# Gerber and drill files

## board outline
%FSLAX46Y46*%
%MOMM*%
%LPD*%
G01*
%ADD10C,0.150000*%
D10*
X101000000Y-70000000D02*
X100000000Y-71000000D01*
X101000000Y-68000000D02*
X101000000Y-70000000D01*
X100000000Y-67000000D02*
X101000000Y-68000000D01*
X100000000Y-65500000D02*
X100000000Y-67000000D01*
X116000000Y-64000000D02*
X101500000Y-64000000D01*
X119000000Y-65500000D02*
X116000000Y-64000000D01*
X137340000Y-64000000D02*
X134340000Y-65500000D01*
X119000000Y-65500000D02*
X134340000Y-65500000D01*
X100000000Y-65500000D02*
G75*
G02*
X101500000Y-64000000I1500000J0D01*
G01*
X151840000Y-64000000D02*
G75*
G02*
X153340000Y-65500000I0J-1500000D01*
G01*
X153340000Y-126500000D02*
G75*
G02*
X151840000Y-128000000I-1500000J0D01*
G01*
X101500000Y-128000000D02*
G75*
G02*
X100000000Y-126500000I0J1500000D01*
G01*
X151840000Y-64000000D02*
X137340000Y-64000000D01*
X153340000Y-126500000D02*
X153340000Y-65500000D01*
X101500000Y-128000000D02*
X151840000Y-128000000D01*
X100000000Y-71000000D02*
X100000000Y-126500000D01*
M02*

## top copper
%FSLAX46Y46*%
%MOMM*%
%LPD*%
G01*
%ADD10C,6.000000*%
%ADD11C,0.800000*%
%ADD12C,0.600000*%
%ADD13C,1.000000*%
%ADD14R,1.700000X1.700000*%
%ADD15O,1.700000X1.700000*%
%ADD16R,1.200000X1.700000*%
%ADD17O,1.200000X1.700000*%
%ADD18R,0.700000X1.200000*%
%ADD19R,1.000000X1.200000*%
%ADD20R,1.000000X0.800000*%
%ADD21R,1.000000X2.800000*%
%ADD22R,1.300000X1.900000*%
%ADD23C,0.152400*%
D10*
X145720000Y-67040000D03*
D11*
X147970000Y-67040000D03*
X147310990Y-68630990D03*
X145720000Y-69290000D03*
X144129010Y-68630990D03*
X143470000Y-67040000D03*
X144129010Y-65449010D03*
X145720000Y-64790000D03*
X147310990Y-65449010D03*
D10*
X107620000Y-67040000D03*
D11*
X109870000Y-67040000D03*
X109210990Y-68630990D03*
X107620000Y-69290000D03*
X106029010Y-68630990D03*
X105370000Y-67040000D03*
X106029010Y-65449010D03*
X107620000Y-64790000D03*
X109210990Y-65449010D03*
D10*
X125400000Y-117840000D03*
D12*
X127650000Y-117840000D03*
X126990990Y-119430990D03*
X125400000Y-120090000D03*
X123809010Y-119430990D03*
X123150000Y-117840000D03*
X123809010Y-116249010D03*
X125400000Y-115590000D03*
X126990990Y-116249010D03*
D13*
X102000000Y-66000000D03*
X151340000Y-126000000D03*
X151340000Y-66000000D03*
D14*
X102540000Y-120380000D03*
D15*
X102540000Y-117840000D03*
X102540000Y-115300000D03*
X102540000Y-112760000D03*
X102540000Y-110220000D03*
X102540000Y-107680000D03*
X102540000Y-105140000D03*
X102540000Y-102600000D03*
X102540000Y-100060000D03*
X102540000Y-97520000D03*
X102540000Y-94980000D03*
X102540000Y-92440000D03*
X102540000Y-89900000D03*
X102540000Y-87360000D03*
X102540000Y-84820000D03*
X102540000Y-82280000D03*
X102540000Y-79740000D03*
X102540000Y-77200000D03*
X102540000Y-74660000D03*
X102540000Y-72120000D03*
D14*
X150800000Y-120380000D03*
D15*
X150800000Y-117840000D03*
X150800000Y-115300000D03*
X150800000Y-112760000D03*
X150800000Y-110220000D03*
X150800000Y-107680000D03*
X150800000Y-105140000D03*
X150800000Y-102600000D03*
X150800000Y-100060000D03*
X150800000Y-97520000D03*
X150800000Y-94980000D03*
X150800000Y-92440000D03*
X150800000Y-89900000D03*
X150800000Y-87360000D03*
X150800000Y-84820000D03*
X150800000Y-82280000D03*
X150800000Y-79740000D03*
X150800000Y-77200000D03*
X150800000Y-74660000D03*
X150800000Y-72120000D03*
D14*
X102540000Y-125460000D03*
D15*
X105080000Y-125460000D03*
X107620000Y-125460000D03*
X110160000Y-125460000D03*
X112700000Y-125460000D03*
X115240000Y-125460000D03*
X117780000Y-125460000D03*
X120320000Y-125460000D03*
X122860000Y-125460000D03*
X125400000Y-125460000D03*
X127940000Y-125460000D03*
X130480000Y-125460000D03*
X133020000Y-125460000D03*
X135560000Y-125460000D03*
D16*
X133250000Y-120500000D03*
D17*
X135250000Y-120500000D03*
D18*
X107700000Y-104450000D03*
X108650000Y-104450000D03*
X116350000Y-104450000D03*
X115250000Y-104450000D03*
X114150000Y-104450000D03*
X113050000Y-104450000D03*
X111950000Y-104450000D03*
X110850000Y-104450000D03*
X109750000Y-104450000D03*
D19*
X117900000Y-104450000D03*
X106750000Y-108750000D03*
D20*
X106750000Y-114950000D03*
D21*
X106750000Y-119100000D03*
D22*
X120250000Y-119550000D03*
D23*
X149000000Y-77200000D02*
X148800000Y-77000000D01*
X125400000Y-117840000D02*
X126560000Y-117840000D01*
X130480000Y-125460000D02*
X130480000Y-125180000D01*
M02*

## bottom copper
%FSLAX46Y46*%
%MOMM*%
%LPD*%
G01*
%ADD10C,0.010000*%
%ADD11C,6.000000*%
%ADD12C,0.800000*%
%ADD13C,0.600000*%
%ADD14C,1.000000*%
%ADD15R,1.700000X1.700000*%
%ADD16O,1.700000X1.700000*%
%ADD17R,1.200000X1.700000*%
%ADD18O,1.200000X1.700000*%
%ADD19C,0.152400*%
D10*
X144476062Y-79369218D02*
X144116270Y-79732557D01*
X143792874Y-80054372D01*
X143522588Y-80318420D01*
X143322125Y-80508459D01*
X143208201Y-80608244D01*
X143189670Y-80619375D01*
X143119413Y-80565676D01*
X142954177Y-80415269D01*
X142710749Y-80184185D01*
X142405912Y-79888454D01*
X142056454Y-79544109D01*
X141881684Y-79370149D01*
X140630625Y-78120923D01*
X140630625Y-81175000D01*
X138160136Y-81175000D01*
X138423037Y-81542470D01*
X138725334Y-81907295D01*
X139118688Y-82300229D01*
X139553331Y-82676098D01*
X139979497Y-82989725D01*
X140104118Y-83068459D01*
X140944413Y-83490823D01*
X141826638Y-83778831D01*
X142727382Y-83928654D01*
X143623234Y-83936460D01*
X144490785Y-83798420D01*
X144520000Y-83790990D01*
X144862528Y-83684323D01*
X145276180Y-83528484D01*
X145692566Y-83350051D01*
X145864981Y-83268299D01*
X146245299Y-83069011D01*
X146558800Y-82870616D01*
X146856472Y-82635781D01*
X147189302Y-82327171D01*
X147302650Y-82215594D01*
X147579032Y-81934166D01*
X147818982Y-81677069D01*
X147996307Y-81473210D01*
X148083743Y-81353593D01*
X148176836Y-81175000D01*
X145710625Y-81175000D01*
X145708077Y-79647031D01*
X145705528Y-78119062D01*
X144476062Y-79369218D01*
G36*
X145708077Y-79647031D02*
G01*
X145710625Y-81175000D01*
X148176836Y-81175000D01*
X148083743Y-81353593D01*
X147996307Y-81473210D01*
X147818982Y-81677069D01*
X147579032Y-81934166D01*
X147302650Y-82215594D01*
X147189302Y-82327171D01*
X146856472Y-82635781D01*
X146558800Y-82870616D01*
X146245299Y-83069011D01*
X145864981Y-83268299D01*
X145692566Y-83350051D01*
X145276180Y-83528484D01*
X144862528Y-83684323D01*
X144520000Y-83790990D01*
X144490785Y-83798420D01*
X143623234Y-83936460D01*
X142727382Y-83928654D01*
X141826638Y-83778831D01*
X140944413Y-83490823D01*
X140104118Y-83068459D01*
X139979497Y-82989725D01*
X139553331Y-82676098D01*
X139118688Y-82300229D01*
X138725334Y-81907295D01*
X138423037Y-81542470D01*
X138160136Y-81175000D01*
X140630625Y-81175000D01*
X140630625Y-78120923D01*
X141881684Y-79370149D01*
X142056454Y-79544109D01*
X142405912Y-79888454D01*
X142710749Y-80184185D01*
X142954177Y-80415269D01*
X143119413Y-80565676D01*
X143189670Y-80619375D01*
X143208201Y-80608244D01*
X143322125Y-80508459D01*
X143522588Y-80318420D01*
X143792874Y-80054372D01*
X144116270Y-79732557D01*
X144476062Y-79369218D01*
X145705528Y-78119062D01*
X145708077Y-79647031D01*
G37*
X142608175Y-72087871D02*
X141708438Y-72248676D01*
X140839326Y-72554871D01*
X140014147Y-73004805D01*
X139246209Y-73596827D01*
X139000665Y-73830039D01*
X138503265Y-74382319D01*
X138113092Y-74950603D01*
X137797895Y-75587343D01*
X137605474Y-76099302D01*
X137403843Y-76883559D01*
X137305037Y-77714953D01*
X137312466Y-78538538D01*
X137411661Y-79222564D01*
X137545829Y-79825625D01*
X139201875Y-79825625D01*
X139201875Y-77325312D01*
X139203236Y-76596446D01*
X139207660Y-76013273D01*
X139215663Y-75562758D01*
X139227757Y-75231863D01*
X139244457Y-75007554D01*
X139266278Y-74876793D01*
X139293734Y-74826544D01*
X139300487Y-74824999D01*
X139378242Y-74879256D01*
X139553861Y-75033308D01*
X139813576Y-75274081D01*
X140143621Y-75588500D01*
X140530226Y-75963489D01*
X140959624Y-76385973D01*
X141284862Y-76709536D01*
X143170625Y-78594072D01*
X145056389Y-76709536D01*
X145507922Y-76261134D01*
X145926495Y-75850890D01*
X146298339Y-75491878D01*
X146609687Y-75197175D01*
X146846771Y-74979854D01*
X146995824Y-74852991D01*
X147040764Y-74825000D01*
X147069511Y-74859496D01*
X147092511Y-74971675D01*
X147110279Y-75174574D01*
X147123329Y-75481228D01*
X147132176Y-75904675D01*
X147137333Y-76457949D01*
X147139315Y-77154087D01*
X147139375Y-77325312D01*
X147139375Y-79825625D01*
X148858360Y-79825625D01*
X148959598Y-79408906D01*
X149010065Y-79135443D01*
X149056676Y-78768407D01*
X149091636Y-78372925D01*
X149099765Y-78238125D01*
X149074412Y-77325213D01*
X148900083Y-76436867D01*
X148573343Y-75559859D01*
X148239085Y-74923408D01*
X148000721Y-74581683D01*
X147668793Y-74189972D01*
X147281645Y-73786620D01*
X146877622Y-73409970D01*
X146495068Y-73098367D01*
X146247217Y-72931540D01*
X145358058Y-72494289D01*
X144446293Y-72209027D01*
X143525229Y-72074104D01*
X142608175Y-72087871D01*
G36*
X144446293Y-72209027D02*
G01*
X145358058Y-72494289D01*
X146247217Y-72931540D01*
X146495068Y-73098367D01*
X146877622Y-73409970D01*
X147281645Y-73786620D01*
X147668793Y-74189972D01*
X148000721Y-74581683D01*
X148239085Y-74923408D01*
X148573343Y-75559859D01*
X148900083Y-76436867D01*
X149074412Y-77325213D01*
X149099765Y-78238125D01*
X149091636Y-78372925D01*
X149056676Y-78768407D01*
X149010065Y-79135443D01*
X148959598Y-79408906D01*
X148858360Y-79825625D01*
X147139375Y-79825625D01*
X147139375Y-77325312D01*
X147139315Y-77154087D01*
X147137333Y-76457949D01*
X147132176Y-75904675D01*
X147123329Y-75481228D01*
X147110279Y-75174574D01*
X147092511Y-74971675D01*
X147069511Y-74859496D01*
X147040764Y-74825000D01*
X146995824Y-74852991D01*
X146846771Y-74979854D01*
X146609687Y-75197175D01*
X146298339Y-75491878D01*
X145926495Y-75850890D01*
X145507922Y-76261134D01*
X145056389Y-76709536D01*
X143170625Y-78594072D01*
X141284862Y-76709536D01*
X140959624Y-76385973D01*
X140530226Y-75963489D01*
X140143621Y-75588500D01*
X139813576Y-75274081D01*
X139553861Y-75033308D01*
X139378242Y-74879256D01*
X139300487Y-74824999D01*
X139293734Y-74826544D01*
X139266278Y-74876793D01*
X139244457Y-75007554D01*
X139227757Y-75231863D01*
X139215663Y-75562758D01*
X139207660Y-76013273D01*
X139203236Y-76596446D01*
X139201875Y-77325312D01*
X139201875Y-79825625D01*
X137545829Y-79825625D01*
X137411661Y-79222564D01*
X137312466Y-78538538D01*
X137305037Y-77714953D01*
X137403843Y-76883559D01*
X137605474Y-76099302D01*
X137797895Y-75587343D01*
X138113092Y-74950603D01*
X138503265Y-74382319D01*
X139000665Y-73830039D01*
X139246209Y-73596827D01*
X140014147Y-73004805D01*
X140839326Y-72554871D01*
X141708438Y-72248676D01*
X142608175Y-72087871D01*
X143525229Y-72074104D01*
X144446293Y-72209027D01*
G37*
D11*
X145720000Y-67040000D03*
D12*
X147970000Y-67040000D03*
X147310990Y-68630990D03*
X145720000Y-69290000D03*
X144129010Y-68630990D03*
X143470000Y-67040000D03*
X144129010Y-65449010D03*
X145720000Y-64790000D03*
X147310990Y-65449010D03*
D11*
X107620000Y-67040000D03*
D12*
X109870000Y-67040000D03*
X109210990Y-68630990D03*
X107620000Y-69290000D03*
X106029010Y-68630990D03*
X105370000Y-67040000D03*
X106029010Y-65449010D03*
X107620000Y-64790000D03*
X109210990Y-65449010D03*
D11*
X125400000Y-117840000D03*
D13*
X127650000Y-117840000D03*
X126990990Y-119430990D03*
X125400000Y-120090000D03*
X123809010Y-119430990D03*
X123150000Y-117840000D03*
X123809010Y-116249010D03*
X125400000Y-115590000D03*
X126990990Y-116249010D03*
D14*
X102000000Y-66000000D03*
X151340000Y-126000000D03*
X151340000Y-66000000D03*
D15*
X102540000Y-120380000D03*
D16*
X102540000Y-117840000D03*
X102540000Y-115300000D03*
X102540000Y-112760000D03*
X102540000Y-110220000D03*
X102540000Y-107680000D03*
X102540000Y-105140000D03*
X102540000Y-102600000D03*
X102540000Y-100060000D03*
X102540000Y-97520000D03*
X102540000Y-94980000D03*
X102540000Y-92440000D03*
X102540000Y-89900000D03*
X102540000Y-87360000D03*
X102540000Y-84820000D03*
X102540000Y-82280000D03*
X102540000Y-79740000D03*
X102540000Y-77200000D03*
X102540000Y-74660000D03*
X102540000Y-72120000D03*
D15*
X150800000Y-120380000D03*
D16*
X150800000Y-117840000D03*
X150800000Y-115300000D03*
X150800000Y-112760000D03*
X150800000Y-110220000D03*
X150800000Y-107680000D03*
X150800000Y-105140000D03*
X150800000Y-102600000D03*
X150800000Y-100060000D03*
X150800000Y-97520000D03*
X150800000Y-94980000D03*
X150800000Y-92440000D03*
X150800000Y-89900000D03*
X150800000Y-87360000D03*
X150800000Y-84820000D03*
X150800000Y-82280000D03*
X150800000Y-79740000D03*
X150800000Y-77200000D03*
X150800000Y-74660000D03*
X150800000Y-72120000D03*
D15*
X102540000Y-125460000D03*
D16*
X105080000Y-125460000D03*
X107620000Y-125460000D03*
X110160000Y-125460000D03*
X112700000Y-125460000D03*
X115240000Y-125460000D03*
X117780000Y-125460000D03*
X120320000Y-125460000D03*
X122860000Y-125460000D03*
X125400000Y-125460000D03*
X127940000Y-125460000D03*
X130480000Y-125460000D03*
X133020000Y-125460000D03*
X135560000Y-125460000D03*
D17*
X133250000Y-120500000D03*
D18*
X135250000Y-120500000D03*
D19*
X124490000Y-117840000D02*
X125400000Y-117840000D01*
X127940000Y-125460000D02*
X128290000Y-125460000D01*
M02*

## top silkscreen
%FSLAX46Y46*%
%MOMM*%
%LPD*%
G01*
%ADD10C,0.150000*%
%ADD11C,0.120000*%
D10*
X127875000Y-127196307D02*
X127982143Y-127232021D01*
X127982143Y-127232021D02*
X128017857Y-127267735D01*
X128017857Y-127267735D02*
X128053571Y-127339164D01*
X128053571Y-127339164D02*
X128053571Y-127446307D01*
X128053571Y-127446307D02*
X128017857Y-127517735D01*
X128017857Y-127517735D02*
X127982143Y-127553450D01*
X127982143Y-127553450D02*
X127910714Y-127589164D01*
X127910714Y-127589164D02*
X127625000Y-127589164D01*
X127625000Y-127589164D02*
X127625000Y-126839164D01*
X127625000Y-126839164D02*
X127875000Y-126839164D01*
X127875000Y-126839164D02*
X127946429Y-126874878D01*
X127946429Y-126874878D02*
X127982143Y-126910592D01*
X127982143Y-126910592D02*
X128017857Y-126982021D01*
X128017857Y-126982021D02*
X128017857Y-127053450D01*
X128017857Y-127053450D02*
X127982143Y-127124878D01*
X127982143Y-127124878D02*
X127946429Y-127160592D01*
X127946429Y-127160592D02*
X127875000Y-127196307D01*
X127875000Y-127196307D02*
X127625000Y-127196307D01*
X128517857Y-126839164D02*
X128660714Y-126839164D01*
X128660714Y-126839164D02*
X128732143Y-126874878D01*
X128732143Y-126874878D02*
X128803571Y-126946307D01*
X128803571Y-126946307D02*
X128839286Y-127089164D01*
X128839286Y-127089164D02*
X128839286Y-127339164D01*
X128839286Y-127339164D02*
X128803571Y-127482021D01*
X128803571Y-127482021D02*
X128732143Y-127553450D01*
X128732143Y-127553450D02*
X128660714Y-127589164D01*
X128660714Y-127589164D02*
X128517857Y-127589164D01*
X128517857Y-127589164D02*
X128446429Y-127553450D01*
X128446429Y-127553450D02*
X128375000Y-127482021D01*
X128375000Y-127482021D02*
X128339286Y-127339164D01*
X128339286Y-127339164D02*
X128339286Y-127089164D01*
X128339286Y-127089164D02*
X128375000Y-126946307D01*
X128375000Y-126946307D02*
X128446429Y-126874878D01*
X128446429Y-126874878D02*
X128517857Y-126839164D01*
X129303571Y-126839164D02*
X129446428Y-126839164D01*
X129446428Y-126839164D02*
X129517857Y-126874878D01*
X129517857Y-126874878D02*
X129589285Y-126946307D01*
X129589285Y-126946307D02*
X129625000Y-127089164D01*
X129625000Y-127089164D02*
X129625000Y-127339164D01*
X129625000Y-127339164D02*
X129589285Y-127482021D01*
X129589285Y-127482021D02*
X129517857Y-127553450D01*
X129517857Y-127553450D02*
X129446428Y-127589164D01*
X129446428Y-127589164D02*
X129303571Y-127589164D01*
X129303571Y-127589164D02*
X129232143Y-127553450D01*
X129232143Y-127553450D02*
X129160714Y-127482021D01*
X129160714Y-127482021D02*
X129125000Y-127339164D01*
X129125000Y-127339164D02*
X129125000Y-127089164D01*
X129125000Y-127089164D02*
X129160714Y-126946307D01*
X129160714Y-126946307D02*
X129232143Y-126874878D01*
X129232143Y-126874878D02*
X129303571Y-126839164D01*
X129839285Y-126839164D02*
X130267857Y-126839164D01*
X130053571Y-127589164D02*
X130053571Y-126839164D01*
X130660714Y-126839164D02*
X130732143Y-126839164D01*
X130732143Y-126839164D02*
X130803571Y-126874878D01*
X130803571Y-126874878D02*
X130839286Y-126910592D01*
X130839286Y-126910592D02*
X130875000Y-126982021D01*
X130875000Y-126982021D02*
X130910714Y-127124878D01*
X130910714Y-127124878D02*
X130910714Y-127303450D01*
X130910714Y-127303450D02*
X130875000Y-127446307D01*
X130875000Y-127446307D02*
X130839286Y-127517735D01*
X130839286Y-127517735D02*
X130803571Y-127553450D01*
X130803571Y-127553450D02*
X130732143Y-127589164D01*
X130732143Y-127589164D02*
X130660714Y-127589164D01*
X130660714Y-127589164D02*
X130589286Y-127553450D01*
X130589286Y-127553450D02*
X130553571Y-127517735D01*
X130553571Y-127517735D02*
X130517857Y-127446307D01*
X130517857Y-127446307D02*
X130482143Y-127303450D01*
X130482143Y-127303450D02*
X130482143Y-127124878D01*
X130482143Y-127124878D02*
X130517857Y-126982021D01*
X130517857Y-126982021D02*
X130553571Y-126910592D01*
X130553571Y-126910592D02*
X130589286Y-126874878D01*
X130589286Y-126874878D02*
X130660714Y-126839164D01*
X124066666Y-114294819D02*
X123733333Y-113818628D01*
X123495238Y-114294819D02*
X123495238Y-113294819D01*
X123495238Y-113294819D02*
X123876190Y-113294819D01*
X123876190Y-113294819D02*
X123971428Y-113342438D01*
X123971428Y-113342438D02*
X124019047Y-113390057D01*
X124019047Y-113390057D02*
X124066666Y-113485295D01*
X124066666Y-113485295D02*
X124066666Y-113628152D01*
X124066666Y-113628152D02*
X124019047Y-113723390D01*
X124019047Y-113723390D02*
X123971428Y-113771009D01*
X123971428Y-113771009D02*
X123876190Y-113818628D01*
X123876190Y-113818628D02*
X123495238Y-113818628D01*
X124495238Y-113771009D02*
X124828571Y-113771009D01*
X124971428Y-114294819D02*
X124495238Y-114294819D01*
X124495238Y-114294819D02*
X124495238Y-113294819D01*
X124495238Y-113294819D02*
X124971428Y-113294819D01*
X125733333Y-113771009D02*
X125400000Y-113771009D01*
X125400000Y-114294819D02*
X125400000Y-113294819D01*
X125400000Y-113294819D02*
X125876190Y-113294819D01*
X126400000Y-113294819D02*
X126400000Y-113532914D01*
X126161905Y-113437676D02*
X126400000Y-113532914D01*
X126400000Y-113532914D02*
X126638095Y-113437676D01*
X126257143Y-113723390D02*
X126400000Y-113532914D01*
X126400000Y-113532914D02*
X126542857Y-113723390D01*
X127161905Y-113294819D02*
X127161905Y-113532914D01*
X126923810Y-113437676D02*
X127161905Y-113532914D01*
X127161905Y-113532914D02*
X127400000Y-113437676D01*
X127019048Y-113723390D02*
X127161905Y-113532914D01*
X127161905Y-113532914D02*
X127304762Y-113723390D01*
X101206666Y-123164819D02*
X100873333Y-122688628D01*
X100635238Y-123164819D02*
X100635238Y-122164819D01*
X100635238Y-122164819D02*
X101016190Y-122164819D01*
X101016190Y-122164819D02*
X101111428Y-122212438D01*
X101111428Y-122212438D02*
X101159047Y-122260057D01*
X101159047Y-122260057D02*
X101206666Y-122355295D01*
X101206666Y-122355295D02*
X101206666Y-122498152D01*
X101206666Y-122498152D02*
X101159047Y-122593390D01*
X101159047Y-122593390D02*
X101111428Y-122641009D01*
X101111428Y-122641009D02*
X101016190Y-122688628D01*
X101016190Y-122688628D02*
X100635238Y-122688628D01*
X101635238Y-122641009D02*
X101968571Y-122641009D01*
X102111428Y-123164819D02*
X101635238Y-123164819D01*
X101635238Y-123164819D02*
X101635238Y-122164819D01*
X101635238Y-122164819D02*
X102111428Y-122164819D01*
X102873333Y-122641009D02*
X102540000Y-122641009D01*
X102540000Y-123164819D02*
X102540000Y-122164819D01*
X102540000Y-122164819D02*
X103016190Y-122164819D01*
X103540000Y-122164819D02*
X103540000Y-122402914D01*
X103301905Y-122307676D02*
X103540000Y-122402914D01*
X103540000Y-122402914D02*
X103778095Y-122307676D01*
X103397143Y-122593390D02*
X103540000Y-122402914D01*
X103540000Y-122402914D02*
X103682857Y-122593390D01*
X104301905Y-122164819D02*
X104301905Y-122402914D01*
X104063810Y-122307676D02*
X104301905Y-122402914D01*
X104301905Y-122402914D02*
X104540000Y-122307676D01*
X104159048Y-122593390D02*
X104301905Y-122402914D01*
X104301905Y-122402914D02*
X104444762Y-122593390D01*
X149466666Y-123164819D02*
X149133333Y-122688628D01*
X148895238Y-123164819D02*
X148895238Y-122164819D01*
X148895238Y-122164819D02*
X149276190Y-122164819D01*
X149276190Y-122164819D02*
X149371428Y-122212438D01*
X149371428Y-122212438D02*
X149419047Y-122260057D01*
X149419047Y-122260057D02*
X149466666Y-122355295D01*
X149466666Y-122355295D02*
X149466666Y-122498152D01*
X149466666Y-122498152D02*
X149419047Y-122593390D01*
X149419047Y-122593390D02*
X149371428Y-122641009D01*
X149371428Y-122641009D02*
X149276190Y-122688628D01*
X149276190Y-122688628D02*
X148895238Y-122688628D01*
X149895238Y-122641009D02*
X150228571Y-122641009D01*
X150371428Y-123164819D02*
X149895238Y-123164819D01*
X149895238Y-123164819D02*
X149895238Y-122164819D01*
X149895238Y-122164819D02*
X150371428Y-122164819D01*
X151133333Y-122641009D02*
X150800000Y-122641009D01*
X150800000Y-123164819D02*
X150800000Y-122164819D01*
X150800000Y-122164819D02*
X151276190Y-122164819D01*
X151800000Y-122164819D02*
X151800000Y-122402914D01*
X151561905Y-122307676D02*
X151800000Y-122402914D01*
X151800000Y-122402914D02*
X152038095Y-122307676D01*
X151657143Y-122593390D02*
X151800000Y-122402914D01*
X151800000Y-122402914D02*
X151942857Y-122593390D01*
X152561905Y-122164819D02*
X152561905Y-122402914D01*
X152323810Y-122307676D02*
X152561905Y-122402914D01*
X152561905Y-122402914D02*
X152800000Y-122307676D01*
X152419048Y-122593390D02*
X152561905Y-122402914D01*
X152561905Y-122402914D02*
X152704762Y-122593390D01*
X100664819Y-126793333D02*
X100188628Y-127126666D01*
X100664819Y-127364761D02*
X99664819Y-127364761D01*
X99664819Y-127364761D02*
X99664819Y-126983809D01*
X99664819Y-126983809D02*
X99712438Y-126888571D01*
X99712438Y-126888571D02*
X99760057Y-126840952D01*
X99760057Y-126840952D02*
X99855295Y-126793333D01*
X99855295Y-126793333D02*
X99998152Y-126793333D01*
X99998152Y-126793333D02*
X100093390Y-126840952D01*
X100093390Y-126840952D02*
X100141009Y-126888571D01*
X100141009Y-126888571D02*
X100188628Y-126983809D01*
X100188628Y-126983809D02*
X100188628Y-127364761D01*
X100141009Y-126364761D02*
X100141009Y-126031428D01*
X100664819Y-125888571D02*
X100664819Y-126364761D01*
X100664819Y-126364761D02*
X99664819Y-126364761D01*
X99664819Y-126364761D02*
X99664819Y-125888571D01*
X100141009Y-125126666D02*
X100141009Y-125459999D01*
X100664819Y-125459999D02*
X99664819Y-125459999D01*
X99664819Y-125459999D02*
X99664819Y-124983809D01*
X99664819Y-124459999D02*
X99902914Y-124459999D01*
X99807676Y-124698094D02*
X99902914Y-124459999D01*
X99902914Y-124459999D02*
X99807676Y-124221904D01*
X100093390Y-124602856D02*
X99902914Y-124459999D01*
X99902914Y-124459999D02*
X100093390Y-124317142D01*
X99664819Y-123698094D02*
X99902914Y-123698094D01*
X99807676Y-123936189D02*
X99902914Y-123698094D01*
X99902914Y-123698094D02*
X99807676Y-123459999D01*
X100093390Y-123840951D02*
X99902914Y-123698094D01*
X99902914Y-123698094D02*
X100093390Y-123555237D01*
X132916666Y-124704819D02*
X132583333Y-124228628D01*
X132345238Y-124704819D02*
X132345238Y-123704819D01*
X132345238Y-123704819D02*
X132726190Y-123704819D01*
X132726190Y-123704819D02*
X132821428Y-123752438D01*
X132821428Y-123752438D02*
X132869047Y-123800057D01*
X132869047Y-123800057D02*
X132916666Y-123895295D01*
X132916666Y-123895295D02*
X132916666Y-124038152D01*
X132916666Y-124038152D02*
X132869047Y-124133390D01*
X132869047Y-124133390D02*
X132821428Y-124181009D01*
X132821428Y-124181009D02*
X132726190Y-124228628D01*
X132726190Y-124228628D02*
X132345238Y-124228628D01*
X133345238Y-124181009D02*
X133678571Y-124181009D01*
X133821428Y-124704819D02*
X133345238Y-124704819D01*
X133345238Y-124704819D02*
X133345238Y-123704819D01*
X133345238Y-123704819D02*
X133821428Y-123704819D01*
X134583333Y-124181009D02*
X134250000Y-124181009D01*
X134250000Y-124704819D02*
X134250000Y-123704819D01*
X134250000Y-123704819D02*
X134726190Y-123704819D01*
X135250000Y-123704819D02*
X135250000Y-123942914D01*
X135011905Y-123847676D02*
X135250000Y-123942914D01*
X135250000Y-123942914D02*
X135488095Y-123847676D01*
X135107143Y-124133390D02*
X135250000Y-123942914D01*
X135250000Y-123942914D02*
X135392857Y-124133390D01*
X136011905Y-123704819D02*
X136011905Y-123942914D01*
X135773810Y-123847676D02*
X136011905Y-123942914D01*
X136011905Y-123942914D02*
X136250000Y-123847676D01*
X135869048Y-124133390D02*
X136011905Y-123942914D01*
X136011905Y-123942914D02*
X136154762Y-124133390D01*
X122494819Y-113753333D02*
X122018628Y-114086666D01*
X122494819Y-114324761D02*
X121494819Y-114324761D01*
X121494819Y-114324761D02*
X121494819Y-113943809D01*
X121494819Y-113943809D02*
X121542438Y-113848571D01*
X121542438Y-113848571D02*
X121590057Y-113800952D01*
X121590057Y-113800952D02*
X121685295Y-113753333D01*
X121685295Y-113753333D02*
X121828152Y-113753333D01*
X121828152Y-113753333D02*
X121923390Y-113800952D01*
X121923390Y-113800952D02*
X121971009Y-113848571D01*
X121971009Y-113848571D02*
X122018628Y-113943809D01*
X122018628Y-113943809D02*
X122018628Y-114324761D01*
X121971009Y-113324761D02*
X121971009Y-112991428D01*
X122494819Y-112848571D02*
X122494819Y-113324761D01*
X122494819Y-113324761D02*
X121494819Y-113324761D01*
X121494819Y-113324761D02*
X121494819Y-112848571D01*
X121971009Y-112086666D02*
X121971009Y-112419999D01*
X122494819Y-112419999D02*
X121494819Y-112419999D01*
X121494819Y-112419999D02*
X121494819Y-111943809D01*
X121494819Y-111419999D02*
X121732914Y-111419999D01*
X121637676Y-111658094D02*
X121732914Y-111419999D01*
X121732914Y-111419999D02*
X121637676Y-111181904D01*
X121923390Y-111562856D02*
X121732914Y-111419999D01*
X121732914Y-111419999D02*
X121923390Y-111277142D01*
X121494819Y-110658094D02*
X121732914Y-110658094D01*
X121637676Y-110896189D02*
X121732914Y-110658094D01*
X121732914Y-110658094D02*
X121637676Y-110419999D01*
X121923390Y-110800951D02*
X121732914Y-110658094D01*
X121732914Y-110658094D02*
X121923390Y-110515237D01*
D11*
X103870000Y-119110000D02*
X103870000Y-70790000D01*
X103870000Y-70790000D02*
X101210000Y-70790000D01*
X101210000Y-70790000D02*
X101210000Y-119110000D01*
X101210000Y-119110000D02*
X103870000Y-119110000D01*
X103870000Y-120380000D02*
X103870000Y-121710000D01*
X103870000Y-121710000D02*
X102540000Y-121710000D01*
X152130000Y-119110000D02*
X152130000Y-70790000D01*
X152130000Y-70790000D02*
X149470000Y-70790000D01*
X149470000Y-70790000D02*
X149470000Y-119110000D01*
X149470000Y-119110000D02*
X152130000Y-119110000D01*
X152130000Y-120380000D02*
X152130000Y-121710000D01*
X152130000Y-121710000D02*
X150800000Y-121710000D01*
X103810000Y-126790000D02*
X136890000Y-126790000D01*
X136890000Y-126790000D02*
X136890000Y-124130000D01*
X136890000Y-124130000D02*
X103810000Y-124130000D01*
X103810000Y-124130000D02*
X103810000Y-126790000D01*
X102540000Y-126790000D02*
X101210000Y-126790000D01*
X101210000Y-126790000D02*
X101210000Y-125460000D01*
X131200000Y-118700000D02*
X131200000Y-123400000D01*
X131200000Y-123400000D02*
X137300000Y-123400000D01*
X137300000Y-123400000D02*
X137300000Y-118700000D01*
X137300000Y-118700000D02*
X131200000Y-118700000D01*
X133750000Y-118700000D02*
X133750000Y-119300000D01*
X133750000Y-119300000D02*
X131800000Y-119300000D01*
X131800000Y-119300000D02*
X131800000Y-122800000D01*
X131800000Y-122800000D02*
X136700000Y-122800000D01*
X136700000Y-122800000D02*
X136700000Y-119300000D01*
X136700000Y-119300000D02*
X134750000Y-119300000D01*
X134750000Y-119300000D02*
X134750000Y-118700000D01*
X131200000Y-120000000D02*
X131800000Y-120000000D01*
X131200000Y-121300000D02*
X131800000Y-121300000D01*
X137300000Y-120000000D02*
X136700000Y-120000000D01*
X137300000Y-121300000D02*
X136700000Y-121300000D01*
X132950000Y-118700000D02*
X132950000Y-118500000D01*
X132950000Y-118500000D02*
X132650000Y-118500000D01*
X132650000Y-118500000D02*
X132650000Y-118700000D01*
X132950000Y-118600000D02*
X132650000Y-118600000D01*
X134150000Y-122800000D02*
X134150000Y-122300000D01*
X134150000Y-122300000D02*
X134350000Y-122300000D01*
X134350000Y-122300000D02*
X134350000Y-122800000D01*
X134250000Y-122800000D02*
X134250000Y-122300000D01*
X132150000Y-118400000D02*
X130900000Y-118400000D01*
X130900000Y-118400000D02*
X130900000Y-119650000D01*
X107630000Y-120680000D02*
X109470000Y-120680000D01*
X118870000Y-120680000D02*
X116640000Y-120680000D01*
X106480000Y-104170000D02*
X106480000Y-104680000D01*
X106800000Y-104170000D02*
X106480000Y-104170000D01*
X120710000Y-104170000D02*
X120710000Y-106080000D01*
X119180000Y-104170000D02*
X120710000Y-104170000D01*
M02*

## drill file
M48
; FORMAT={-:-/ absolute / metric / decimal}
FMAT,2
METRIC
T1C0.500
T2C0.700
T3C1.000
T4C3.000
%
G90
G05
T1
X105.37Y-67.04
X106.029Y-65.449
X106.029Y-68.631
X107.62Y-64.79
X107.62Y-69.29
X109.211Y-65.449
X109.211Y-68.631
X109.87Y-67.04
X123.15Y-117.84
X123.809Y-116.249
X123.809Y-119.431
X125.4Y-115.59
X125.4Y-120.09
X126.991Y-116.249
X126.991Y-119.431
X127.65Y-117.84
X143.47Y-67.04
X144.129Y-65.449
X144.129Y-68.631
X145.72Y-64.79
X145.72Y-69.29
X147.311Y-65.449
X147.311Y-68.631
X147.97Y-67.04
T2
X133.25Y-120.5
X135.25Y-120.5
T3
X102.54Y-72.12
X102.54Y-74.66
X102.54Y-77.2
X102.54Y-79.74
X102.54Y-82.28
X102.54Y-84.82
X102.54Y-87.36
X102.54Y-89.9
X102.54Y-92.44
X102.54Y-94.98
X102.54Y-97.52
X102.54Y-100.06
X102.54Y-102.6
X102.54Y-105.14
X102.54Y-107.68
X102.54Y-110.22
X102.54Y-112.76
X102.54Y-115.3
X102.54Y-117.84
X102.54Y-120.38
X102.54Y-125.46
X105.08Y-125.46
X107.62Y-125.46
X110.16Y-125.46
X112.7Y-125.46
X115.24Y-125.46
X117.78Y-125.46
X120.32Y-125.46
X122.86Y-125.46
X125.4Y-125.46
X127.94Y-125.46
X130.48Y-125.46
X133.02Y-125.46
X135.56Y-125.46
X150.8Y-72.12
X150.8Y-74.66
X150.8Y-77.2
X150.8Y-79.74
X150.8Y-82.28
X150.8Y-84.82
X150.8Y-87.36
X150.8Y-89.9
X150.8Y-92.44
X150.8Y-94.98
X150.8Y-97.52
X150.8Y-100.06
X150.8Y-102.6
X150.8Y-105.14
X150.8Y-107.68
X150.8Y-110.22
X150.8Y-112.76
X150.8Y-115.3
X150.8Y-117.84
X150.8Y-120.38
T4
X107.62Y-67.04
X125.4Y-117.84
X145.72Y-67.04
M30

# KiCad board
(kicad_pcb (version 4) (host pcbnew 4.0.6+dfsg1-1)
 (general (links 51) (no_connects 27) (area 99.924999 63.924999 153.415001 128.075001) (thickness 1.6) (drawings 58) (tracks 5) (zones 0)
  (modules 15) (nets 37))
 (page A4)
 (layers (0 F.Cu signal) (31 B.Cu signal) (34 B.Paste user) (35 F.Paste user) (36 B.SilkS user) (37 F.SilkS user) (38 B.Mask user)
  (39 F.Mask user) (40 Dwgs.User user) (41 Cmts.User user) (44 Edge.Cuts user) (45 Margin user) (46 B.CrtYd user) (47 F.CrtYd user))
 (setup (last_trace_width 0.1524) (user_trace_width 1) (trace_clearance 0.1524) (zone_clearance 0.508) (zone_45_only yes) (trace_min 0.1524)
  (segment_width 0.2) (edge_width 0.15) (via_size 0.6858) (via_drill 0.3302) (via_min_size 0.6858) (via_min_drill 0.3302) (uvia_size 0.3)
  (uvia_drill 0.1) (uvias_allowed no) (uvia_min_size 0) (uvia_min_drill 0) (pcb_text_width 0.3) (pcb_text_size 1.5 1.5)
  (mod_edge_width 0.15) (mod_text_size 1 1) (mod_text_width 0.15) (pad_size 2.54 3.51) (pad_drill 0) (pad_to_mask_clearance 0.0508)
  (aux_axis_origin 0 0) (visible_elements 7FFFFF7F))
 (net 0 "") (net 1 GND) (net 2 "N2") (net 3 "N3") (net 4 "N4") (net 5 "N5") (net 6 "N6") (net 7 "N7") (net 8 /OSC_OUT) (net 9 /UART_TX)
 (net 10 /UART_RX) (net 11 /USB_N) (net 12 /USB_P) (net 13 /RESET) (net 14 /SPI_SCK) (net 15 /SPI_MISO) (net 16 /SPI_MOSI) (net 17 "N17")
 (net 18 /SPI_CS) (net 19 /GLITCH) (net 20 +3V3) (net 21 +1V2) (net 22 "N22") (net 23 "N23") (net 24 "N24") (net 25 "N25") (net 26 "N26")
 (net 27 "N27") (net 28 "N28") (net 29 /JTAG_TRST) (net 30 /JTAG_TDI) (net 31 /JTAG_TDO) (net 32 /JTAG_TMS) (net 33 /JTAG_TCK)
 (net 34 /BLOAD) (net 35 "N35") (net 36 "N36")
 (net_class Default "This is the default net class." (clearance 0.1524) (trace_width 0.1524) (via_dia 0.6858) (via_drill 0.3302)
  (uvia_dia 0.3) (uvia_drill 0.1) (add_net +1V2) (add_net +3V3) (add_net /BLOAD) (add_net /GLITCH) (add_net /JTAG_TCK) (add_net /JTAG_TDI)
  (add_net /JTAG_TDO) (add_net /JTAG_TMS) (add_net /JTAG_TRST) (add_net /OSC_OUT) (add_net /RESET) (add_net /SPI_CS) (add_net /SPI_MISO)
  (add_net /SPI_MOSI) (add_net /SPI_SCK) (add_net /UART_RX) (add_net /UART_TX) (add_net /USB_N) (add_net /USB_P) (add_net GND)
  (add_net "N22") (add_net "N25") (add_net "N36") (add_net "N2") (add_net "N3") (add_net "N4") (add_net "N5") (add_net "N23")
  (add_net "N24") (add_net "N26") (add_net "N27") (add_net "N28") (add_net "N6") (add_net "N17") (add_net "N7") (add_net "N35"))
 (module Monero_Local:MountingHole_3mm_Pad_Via (layer F.Cu) (at 145.72 67.04)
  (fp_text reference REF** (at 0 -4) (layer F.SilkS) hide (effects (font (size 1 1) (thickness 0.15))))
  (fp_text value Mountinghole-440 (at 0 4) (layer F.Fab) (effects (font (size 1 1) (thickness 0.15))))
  (pad 1 thru_hole circle (at 0 0) (size 6 6) (drill 3) (layers *.Cu *.Mask) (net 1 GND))
  (pad 1 thru_hole circle (at 2.25 0) (size 0.8 0.8) (drill 0.5) (layers *.Cu *.Mask) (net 1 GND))
  (pad 1 thru_hole circle (at 1.59099 1.59099) (size 0.8 0.8) (drill 0.5) (layers *.Cu *.Mask) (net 1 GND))
  (pad 1 thru_hole circle (at 0 2.25) (size 0.8 0.8) (drill 0.5) (layers *.Cu *.Mask) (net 1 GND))
  (pad 1 thru_hole circle (at -1.59099 1.59099) (size 0.8 0.8) (drill 0.5) (layers *.Cu *.Mask) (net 1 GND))
  (pad 1 thru_hole circle (at -2.25 0) (size 0.8 0.8) (drill 0.5) (layers *.Cu *.Mask) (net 1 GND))
  (pad 1 thru_hole circle (at -1.59099 -1.59099) (size 0.8 0.8) (drill 0.5) (layers *.Cu *.Mask) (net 1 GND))
  (pad 1 thru_hole circle (at 0 -2.25) (size 0.8 0.8) (drill 0.5) (layers *.Cu *.Mask) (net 1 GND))
  (pad 1 thru_hole circle (at 1.59099 -1.59099) (size 0.8 0.8) (drill 0.5) (layers *.Cu *.Mask) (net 1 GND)))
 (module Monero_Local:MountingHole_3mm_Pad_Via (layer F.Cu) (at 107.62 67.04)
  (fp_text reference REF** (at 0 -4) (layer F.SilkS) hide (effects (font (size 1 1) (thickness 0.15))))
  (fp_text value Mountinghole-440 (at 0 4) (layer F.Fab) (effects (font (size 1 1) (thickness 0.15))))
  (pad 1 thru_hole circle (at 0 0) (size 6 6) (drill 3) (layers *.Cu *.Mask) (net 1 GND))
  (pad 1 thru_hole circle (at 2.25 0) (size 0.8 0.8) (drill 0.5) (layers *.Cu *.Mask) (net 1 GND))
  (pad 1 thru_hole circle (at 1.59099 1.59099) (size 0.8 0.8) (drill 0.5) (layers *.Cu *.Mask) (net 1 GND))
  (pad 1 thru_hole circle (at 0 2.25) (size 0.8 0.8) (drill 0.5) (layers *.Cu *.Mask) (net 1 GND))
  (pad 1 thru_hole circle (at -1.59099 1.59099) (size 0.8 0.8) (drill 0.5) (layers *.Cu *.Mask) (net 1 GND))
  (pad 1 thru_hole circle (at -2.25 0) (size 0.8 0.8) (drill 0.5) (layers *.Cu *.Mask) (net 1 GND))
  (pad 1 thru_hole circle (at -1.59099 -1.59099) (size 0.8 0.8) (drill 0.5) (layers *.Cu *.Mask) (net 1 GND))
  (pad 1 thru_hole circle (at 0 -2.25) (size 0.8 0.8) (drill 0.5) (layers *.Cu *.Mask) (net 1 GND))
  (pad 1 thru_hole circle (at 1.59099 -1.59099) (size 0.8 0.8) (drill 0.5) (layers *.Cu *.Mask) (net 1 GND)))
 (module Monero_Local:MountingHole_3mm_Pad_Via (layer F.Cu) (at 125.4 117.84)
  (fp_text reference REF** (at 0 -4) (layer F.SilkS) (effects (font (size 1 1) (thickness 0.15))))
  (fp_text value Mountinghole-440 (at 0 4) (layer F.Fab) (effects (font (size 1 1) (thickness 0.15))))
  (pad 1 thru_hole circle (at 0 0) (size 6 6) (drill 3) (layers *.Cu *.Mask) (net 1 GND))
  (pad 1 thru_hole circle (at 2.25 0) (size 0.6 0.6) (drill 0.5) (layers *.Cu *.Mask) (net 1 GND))
  (pad 1 thru_hole circle (at 1.59099 1.59099) (size 0.6 0.6) (drill 0.5) (layers *.Cu *.Mask) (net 1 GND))
  (pad 1 thru_hole circle (at 0 2.25) (size 0.6 0.6) (drill 0.5) (layers *.Cu *.Mask) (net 1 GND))
  (pad 1 thru_hole circle (at -1.59099 1.59099) (size 0.6 0.6) (drill 0.5) (layers *.Cu *.Mask) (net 1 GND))
  (pad 1 thru_hole circle (at -2.25 0) (size 0.6 0.6) (drill 0.5) (layers *.Cu *.Mask) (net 1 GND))
  (pad 1 thru_hole circle (at -1.59099 -1.59099) (size 0.6 0.6) (drill 0.5) (layers *.Cu *.Mask) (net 1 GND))
  (pad 1 thru_hole circle (at 0 -2.25) (size 0.6 0.6) (drill 0.5) (layers *.Cu *.Mask) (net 1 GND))
  (pad 1 thru_hole circle (at 1.59099 -1.59099) (size 0.6 0.6) (drill 0.5) (layers *.Cu *.Mask) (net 1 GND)))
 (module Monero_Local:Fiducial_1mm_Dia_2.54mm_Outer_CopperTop (layer F.Cu) (at 102 66)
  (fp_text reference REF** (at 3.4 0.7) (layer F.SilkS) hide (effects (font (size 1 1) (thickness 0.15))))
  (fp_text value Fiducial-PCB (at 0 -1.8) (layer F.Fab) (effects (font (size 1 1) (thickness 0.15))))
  (pad ~ smd circle (at 0 0) (size 1 1) (layers F.Cu F.Mask) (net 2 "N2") (solder_mask_margin 0.77) (clearance 0.77)))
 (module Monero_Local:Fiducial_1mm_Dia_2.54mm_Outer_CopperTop (layer F.Cu) (at 151.34 126)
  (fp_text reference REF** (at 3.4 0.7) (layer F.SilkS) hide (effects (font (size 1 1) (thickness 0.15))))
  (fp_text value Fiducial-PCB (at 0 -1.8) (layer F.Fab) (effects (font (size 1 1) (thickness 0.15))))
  (pad ~ smd circle (at 0 0) (size 1 1) (layers F.Cu F.Mask) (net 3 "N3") (solder_mask_margin 0.77) (clearance 0.77)))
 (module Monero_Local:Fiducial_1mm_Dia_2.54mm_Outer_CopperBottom (layer F.Cu) (at 102 66)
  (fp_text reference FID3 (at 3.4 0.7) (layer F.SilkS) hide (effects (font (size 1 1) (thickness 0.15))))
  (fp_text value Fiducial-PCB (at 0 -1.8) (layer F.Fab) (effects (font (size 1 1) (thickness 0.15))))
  (pad ~ smd circle (at 0 0) (size 1 1) (layers B.Cu B.Mask) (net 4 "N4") (solder_mask_margin 0.77) (clearance 0.77)))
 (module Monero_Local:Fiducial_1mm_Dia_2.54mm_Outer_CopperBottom (layer F.Cu) (at 151.34 126)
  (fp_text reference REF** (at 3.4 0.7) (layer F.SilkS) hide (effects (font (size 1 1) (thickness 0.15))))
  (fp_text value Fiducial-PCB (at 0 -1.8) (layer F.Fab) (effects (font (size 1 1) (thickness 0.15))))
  (pad ~ smd circle (at 0 0) (size 1 1) (layers B.Cu B.Mask) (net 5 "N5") (solder_mask_margin 0.77) (clearance 0.77)))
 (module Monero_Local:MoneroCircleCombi (layer B.Cu) (at 143.25 78 180)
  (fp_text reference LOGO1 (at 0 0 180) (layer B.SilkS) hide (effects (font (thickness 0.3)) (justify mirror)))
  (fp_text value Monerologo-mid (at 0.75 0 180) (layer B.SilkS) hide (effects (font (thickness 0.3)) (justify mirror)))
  (fp_poly
   (pts (xy -1.226062 -1.369218) (xy -0.86627 -1.732557) (xy -0.542874 -2.054372) (xy -0.272588 -2.31842) (xy -0.072125 -2.508459)
    (xy 0.041799 -2.608244) (xy 0.06033 -2.619375) (xy 0.130587 -2.565676) (xy 0.295823 -2.415269) (xy 0.539251 -2.184185)
    (xy 0.844088 -1.888454) (xy 1.193546 -1.544109) (xy 1.368316 -1.370149) (xy 2.619375 -0.120923) (xy 2.619375 -3.175)
    (xy 5.089864 -3.175) (xy 4.826963 -3.54247) (xy 4.524666 -3.907295) (xy 4.131312 -4.300229) (xy 3.696669 -4.676098)
    (xy 3.270503 -4.989725) (xy 3.145882 -5.068459) (xy 2.305587 -5.490823) (xy 1.423362 -5.778831) (xy 0.522618 -5.928654)
    (xy -0.373234 -5.93646) (xy -1.240785 -5.79842) (xy -1.27 -5.79099) (xy -1.612528 -5.684323) (xy -2.02618 -5.528484)
    (xy -2.442566 -5.350051) (xy -2.614981 -5.268299) (xy -2.995299 -5.069011) (xy -3.3088 -4.870616) (xy -3.606472 -4.635781)
    (xy -3.939302 -4.327171) (xy -4.05265 -4.215594) (xy -4.329032 -3.934166) (xy -4.568982 -3.677069) (xy -4.746307 -3.47321)
    (xy -4.833743 -3.353593) (xy -4.926836 -3.175) (xy -2.460625 -3.175) (xy -2.458077 -1.647031) (xy -2.455528 -0.119062)
    (xy -1.226062 -1.369218))
   (layer B.Cu) (width 0.01))
  (fp_poly
   (pts (xy 0.641825 5.912129) (xy 1.541562 5.751324) (xy 2.410674 5.445129) (xy 3.235853 4.995195) (xy 4.003791 4.403173)
    (xy 4.249335 4.169961) (xy 4.746735 3.617681) (xy 5.136908 3.049397) (xy 5.452105 2.412657) (xy 5.644526 1.900698)
    (xy 5.846157 1.116441) (xy 5.944963 0.285047) (xy 5.937534 -0.538538) (xy 5.838339 -1.222564) (xy 5.704171 -1.825625)
    (xy 4.048125 -1.825625) (xy 4.048125 0.674688) (xy 4.046764 1.403554) (xy 4.04234 1.986727) (xy 4.034337 2.437242)
    (xy 4.022243 2.768137) (xy 4.005543 2.992446) (xy 3.983722 3.123207) (xy 3.956266 3.173456) (xy 3.949513 3.175001)
    (xy 3.871758 3.120744) (xy 3.696139 2.966692) (xy 3.436424 2.725919) (xy 3.106379 2.4115) (xy 2.719774 2.036511) (xy 2.290376 1.614027)
    (xy 1.965138 1.290464) (xy 0.079375 -0.594072) (xy -1.806389 1.290464) (xy -2.257922 1.738866) (xy -2.676495 2.14911)
    (xy -3.048339 2.508122) (xy -3.359687 2.802825) (xy -3.596771 3.020146) (xy -3.745824 3.147009) (xy -3.790764 3.175)
    (xy -3.819511 3.140504) (xy -3.842511 3.028325) (xy -3.860279 2.825426) (xy -3.873329 2.518772) (xy -3.882176 2.095325)
    (xy -3.887333 1.542051) (xy -3.889315 0.845913) (xy -3.889375 0.674688) (xy -3.889375 -1.825625) (xy -5.60836 -1.825625)
    (xy -5.709598 -1.408906) (xy -5.760065 -1.135443) (xy -5.806676 -0.768407) (xy -5.841636 -0.372925) (xy -5.849765 -0.238125)
    (xy -5.824412 0.674787) (xy -5.650083 1.563133) (xy -5.323343 2.440141) (xy -4.989085 3.076592) (xy -4.750721 3.418317)
    (xy -4.418793 3.810028) (xy -4.031645 4.21338) (xy -3.627622 4.59003) (xy -3.245068 4.901633) (xy -2.997217 5.06846)
    (xy -2.108058 5.505711) (xy -1.196293 5.790973) (xy -0.275229 5.925896) (xy 0.641825 5.912129))
   (layer B.Cu) (width 0.01)))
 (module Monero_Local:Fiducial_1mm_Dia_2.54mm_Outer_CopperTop (layer B.Cu) (at 151.34 66)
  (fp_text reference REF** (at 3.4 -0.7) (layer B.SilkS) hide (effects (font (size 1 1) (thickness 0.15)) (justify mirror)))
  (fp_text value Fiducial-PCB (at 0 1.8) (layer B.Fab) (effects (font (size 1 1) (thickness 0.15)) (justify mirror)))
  (pad ~ smd circle (at 0 0) (size 1 1) (layers B.Cu B.Mask) (solder_mask_margin 0.77) (clearance 0.77)))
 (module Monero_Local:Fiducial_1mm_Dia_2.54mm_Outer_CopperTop (layer F.Cu) (at 151.34 66)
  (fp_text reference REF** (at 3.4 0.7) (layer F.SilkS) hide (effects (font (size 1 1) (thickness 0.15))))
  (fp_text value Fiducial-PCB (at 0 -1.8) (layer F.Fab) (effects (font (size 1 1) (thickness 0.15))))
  (pad ~ smd circle (at 0 0) (size 1 1) (layers F.Cu F.Mask) (solder_mask_margin 0.77) (clearance 0.77)))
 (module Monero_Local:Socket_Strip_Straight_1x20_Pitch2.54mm (layer F.Cu) (at 102.54 120.38 180)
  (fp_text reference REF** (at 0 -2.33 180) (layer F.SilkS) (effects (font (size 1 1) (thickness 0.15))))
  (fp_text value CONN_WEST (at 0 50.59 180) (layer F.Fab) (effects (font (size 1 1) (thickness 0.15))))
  (fp_line (start -1.33 1.27) (end -1.33 49.59) (layer F.SilkS) (width 0.12))
  (fp_line (start -1.33 49.59) (end 1.33 49.59) (layer F.SilkS) (width 0.12))
  (fp_line (start 1.33 49.59) (end 1.33 1.27) (layer F.SilkS) (width 0.12))
  (fp_line (start 1.33 1.27) (end -1.33 1.27) (layer F.SilkS) (width 0.12))
  (fp_line (start -1.33 0) (end -1.33 -1.33) (layer F.SilkS) (width 0.12))
  (fp_line (start -1.33 -1.33) (end 0 -1.33) (layer F.SilkS) (width 0.12))
  (pad 1 thru_hole rect (at 0 0 180) (size 1.7 1.7) (drill 1) (layers *.Cu *.Mask) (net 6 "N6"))
  (pad 2 thru_hole oval (at 0 2.54 180) (size 1.7 1.7) (drill 1) (layers *.Cu *.Mask) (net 1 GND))
  (pad 3 thru_hole oval (at 0 5.08 180) (size 1.7 1.7) (drill 1) (layers *.Cu *.Mask) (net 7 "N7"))
  (pad 4 thru_hole oval (at 0 7.62 180) (size 1.7 1.7) (drill 1) (layers *.Cu *.Mask) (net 1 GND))
  (pad 5 thru_hole oval (at 0 10.16 180) (size 1.7 1.7) (drill 1) (layers *.Cu *.Mask) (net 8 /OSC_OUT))
  (pad 6 thru_hole oval (at 0 12.7 180) (size 1.7 1.7) (drill 1) (layers *.Cu *.Mask) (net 1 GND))
  (pad 7 thru_hole oval (at 0 15.24 180) (size 1.7 1.7) (drill 1) (layers *.Cu *.Mask) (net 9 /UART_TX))
  (pad 8 thru_hole oval (at 0 17.78 180) (size 1.7 1.7) (drill 1) (layers *.Cu *.Mask) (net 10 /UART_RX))
  (pad 9 thru_hole oval (at 0 20.32 180) (size 1.7 1.7) (drill 1) (layers *.Cu *.Mask) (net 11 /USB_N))
  (pad 10 thru_hole oval (at 0 22.86 180) (size 1.7 1.7) (drill 1) (layers *.Cu *.Mask) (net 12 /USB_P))
  (pad 11 thru_hole oval (at 0 25.4 180) (size 1.7 1.7) (drill 1) (layers *.Cu *.Mask) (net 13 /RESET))
  (pad 12 thru_hole oval (at 0 27.94 180) (size 1.7 1.7) (drill 1) (layers *.Cu *.Mask) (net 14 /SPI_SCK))
  (pad 13 thru_hole oval (at 0 30.48 180) (size 1.7 1.7) (drill 1) (layers *.Cu *.Mask) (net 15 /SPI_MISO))
  (pad 14 thru_hole oval (at 0 33.02 180) (size 1.7 1.7) (drill 1) (layers *.Cu *.Mask) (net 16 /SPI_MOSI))
  (pad 15 thru_hole oval (at 0 35.56 180) (size 1.7 1.7) (drill 1) (layers *.Cu *.Mask) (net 1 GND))
  (pad 16 thru_hole oval (at 0 38.1 180) (size 1.7 1.7) (drill 1) (layers *.Cu *.Mask) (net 1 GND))
  (pad 17 thru_hole oval (at 0 40.64 180) (size 1.7 1.7) (drill 1) (layers *.Cu *.Mask) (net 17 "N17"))
  (pad 18 thru_hole oval (at 0 43.18 180) (size 1.7 1.7) (drill 1) (layers *.Cu *.Mask) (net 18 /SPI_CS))
  (pad 19 thru_hole oval (at 0 45.72 180) (size 1.7 1.7) (drill 1) (layers *.Cu *.Mask) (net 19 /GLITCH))
  (pad 20 thru_hole oval (at 0 48.26 180) (size 1.7 1.7) (drill 1) (layers *.Cu *.Mask) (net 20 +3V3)))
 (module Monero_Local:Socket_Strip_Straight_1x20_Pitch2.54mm (layer F.Cu) (at 150.8 120.38 180)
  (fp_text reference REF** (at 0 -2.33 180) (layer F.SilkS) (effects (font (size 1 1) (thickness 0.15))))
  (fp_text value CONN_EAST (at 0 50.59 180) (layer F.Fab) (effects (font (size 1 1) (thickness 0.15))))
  (fp_line (start -1.33 1.27) (end -1.33 49.59) (layer F.SilkS) (width 0.12))
  (fp_line (start -1.33 49.59) (end 1.33 49.59) (layer F.SilkS) (width 0.12))
  (fp_line (start 1.33 49.59) (end 1.33 1.27) (layer F.SilkS) (width 0.12))
  (fp_line (start 1.33 1.27) (end -1.33 1.27) (layer F.SilkS) (width 0.12))
  (fp_line (start -1.33 0) (end -1.33 -1.33) (layer F.SilkS) (width 0.12))
  (fp_line (start -1.33 -1.33) (end 0 -1.33) (layer F.SilkS) (width 0.12))
  (pad 1 thru_hole rect (at 0 0 180) (size 1.7 1.7) (drill 1) (layers *.Cu *.Mask) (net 1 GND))
  (pad 2 thru_hole oval (at 0 2.54 180) (size 1.7 1.7) (drill 1) (layers *.Cu *.Mask) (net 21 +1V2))
  (pad 3 thru_hole oval (at 0 5.08 180) (size 1.7 1.7) (drill 1) (layers *.Cu *.Mask) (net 21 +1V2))
  (pad 4 thru_hole oval (at 0 7.62 180) (size 1.7 1.7) (drill 1) (layers *.Cu *.Mask) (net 1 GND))
  (pad 5 thru_hole oval (at 0 10.16 180) (size 1.7 1.7) (drill 1) (layers *.Cu *.Mask) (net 21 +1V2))
  (pad 6 thru_hole oval (at 0 12.7 180) (size 1.7 1.7) (drill 1) (layers *.Cu *.Mask) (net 21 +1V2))
  (pad 7 thru_hole oval (at 0 15.24 180) (size 1.7 1.7) (drill 1) (layers *.Cu *.Mask) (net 1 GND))
  (pad 8 thru_hole oval (at 0 17.78 180) (size 1.7 1.7) (drill 1) (layers *.Cu *.Mask) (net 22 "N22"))
  (pad 9 thru_hole oval (at 0 20.32 180) (size 1.7 1.7) (drill 1) (layers *.Cu *.Mask) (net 1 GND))
  (pad 10 thru_hole oval (at 0 22.86 180) (size 1.7 1.7) (drill 1) (layers *.Cu *.Mask) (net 1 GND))
  (pad 11 thru_hole oval (at 0 25.4 180) (size 1.7 1.7) (drill 1) (layers *.Cu *.Mask) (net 22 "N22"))
  (pad 12 thru_hole oval (at 0 27.94 180) (size 1.7 1.7) (drill 1) (layers *.Cu *.Mask) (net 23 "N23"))
  (pad 13 thru_hole oval (at 0 30.48 180) (size 1.7 1.7) (drill 1) (layers *.Cu *.Mask) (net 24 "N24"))
  (pad 14 thru_hole oval (at 0 33.02 180) (size 1.7 1.7) (drill 1) (layers *.Cu *.Mask) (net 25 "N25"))
  (pad 15 thru_hole oval (at 0 35.56 180) (size 1.7 1.7) (drill 1) (layers *.Cu *.Mask) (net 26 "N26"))
  (pad 16 thru_hole oval (at 0 38.1 180) (size 1.7 1.7) (drill 1) (layers *.Cu *.Mask) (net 1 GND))
  (pad 17 thru_hole oval (at 0 40.64 180) (size 1.7 1.7) (drill 1) (layers *.Cu *.Mask) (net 1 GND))
  (pad 18 thru_hole oval (at 0 43.18 180) (size 1.7 1.7) (drill 1) (layers *.Cu *.Mask) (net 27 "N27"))
  (pad 19 thru_hole oval (at 0 45.72 180) (size 1.7 1.7) (drill 1) (layers *.Cu *.Mask) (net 1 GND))
  (pad 20 thru_hole oval (at 0 48.26 180) (size 1.7 1.7) (drill 1) (layers *.Cu *.Mask) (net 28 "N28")))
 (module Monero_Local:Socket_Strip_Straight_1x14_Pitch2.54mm (layer F.Cu) (at 102.54 125.46 90)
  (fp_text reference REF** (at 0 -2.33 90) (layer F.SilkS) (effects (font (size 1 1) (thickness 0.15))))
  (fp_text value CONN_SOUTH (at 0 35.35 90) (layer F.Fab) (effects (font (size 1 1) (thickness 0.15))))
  (fp_line (start -1.33 1.27) (end -1.33 34.35) (layer F.SilkS) (width 0.12))
  (fp_line (start -1.33 34.35) (end 1.33 34.35) (layer F.SilkS) (width 0.12))
  (fp_line (start 1.33 34.35) (end 1.33 1.27) (layer F.SilkS) (width 0.12))
  (fp_line (start 1.33 1.27) (end -1.33 1.27) (layer F.SilkS) (width 0.12))
  (fp_line (start -1.33 0) (end -1.33 -1.33) (layer F.SilkS) (width 0.12))
  (fp_line (start -1.33 -1.33) (end 0 -1.33) (layer F.SilkS) (width 0.12))
  (pad 1 thru_hole rect (at 0 0 90) (size 1.7 1.7) (drill 1) (layers *.Cu *.Mask) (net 1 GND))
  (pad 2 thru_hole oval (at 0 2.54 90) (size 1.7 1.7) (drill 1) (layers *.Cu *.Mask) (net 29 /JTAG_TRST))
  (pad 3 thru_hole oval (at 0 5.08 90) (size 1.7 1.7) (drill 1) (layers *.Cu *.Mask) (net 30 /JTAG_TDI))
  (pad 4 thru_hole oval (at 0 7.62 90) (size 1.7 1.7) (drill 1) (layers *.Cu *.Mask) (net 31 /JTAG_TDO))
  (pad 5 thru_hole oval (at 0 10.16 90) (size 1.7 1.7) (drill 1) (layers *.Cu *.Mask) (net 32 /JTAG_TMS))
  (pad 6 thru_hole oval (at 0 12.7 90) (size 1.7 1.7) (drill 1) (layers *.Cu *.Mask) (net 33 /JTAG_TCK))
  (pad 7 thru_hole oval (at 0 15.24 90) (size 1.7 1.7) (drill 1) (layers *.Cu *.Mask) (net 20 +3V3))
  (pad 8 thru_hole oval (at 0 17.78 90) (size 1.7 1.7) (drill 1) (layers *.Cu *.Mask) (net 13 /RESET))
  (pad 9 thru_hole oval (at 0 20.32 90) (size 1.7 1.7) (drill 1) (layers *.Cu *.Mask) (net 1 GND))
  (pad 10 thru_hole oval (at 0 22.86 90) (size 1.7 1.7) (drill 1) (layers *.Cu *.Mask) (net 1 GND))
  (pad 11 thru_hole oval (at 0 25.4 90) (size 1.7 1.7) (drill 1) (layers *.Cu *.Mask) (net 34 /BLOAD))
  (pad 12 thru_hole oval (at 0 27.94 90) (size 1.7 1.7) (drill 1) (layers *.Cu *.Mask) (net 20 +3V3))
  (pad 13 thru_hole oval (at 0 30.48 90) (size 1.7 1.7) (drill 1) (layers *.Cu *.Mask) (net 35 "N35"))
  (pad 14 thru_hole oval (at 0 33.02 90) (size 1.7 1.7) (drill 1) (layers *.Cu *.Mask) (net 20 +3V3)))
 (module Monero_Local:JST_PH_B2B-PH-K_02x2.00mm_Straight (layer F.Cu) (at 133.25 120.5)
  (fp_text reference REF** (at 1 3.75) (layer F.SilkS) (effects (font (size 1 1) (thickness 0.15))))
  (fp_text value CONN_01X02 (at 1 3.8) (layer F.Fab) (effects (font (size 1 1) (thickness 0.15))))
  (fp_line (start -2.05 -1.8) (end -2.05 2.9) (layer F.SilkS) (width 0.12))
  (fp_line (start -2.05 2.9) (end 4.05 2.9) (layer F.SilkS) (width 0.12))
  (fp_line (start 4.05 2.9) (end 4.05 -1.8) (layer F.SilkS) (width 0.12))
  (fp_line (start 4.05 -1.8) (end -2.05 -1.8) (layer F.SilkS) (width 0.12))
  (fp_line (start 0.5 -1.8) (end 0.5 -1.2) (layer F.SilkS) (width 0.12))
  (fp_line (start 0.5 -1.2) (end -1.45 -1.2) (layer F.SilkS) (width 0.12))
  (fp_line (start -1.45 -1.2) (end -1.45 2.3) (layer F.SilkS) (width 0.12))
  (fp_line (start -1.45 2.3) (end 3.45 2.3) (layer F.SilkS) (width 0.12))
  (fp_line (start 3.45 2.3) (end 3.45 -1.2) (layer F.SilkS) (width 0.12))
  (fp_line (start 3.45 -1.2) (end 1.5 -1.2) (layer F.SilkS) (width 0.12))
  (fp_line (start 1.5 -1.2) (end 1.5 -1.8) (layer F.SilkS) (width 0.12))
  (fp_line (start -2.05 -0.5) (end -1.45 -0.5) (layer F.SilkS) (width 0.12))
  (fp_line (start -2.05 0.8) (end -1.45 0.8) (layer F.SilkS) (width 0.12))
  (fp_line (start 4.05 -0.5) (end 3.45 -0.5) (layer F.SilkS) (width 0.12))
  (fp_line (start 4.05 0.8) (end 3.45 0.8) (layer F.SilkS) (width 0.12))
  (fp_line (start -0.3 -1.8) (end -0.3 -2) (layer F.SilkS) (width 0.12))
  (fp_line (start -0.3 -2) (end -0.6 -2) (layer F.SilkS) (width 0.12))
  (fp_line (start -0.6 -2) (end -0.6 -1.8) (layer F.SilkS) (width 0.12))
  (fp_line (start -0.3 -1.9) (end -0.6 -1.9) (layer F.SilkS) (width 0.12))
  (fp_line (start 0.9 2.3) (end 0.9 1.8) (layer F.SilkS) (width 0.12))
  (fp_line (start 0.9 1.8) (end 1.1 1.8) (layer F.SilkS) (width 0.12))
  (fp_line (start 1.1 1.8) (end 1.1 2.3) (layer F.SilkS) (width 0.12))
  (fp_line (start 1 2.3) (end 1 1.8) (layer F.SilkS) (width 0.12))
  (fp_line (start -1.1 -2.1) (end -2.35 -2.1) (layer F.SilkS) (width 0.12))
  (fp_line (start -2.35 -2.1) (end -2.35 -0.85) (layer F.SilkS) (width 0.12))
  (pad 1 thru_hole rect (at 0 0) (size 1.2 1.7) (drill 0.7) (layers *.Cu *.Mask) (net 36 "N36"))
  (pad 2 thru_hole oval (at 2 0) (size 1.2 1.7) (drill 0.7) (layers *.Cu *.Mask) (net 1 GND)))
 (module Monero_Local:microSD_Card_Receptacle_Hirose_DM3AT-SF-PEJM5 (layer F.Cu) (at 113.5 112)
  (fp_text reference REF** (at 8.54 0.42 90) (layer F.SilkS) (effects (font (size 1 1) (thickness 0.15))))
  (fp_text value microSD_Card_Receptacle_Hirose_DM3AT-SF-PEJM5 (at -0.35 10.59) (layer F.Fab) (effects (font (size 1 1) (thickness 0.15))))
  (fp_line (start -5.87 8.68) (end -4.03 8.68) (layer F.SilkS) (width 0.12))
  (fp_line (start 5.37 8.68) (end 3.14 8.68) (layer F.SilkS) (width 0.12))
  (fp_line (start -7.02 -7.83) (end -7.02 -7.32) (layer F.SilkS) (width 0.12))
  (fp_line (start -6.7 -7.83) (end -7.02 -7.83) (layer F.SilkS) (width 0.12))
  (fp_line (start 7.21 -7.83) (end 7.21 -5.92) (layer F.SilkS) (width 0.12))
  (fp_line (start 5.68 -7.83) (end 7.21 -7.83) (layer F.SilkS) (width 0.12))
  (pad 9 smd rect (at -5.8 -7.55) (size 0.7 1.2) (layers F.Cu F.Paste F.Mask))
  (pad 8 smd rect (at -4.85 -7.55) (size 0.7 1.2) (layers F.Cu F.Paste F.Mask))
  (pad 1 smd rect (at 2.85 -7.55) (size 0.7 1.2) (layers F.Cu F.Paste F.Mask))
  (pad 2 smd rect (at 1.75 -7.55) (size 0.7 1.2) (layers F.Cu F.Paste F.Mask))
  (pad 3 smd rect (at 0.65 -7.55) (size 0.7 1.2) (layers F.Cu F.Paste F.Mask))
  (pad 4 smd rect (at -0.45 -7.55) (size 0.7 1.2) (layers F.Cu F.Paste F.Mask))
  (pad 5 smd rect (at -1.55 -7.55) (size 0.7 1.2) (layers F.Cu F.Paste F.Mask))
  (pad 6 smd rect (at -2.65 -7.55) (size 0.7 1.2) (layers F.Cu F.Paste F.Mask))
  (pad 7 smd rect (at -3.75 -7.55) (size 0.7 1.2) (layers F.Cu F.Paste F.Mask))
  (pad 11 smd rect (at 4.4 -7.55) (size 1 1.2) (layers F.Cu F.Paste F.Mask))
  (pad 11 smd rect (at -6.75 -3.25) (size 1 1.2) (layers F.Cu F.Paste F.Mask))
  (pad 10 smd rect (at -6.75 2.95) (size 1 0.8) (layers F.Cu F.Paste F.Mask))
  (pad 11 smd rect (at -6.75 7.1) (size 1 2.8) (layers F.Cu F.Paste F.Mask))
  (pad 11 smd rect (at 6.75 7.55) (size 1.3 1.9) (layers F.Cu F.Paste F.Mask)))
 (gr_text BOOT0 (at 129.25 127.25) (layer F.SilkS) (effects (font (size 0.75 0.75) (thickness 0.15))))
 (gr_line (start 101 70) (end 100 71) (angle 90) (layer Edge.Cuts) (width 0.15))
 (gr_line (start 101 68) (end 101 70) (angle 90) (layer Edge.Cuts) (width 0.15))
 (gr_line (start 100 67) (end 101 68) (angle 90) (layer Edge.Cuts) (width 0.15))
 (gr_line (start 100 65.5) (end 100 67) (angle 90) (layer Edge.Cuts) (width 0.15))
 (gr_line (start 116 64) (end 101.5 64) (angle 90) (layer Edge.Cuts) (width 0.15))
 (gr_line (start 119 65.5) (end 116 64) (angle 90) (layer Edge.Cuts) (width 0.15))
 (gr_line (start 137.34 64) (end 134.34 65.5) (angle 90) (layer Edge.Cuts) (width 0.15))
 (gr_line (start 119 65.5) (end 134.34 65.5) (angle 90) (layer Edge.Cuts) (width 0.15))
 (gr_arc (start 101.5 65.5) (end 100 65.5) (angle 90) (layer Edge.Cuts) (width 0.15))
 (gr_arc (start 151.84 65.5) (end 151.84 64) (angle 90) (layer Edge.Cuts) (width 0.15))
 (gr_arc (start 151.84 126.5) (end 153.34 126.5) (angle 90) (layer Edge.Cuts) (width 0.15))
 (gr_arc (start 101.5 126.5) (end 101.5 128) (angle 90) (layer Edge.Cuts) (width 0.15))
 (gr_line (start 151.84 64) (end 137.34 64) (angle 90) (layer Edge.Cuts) (width 0.15))
 (gr_line (start 153.34 126.5) (end 153.34 65.5) (angle 90) (layer Edge.Cuts) (width 0.15))
 (gr_line (start 101.5 128) (end 151.84 128) (angle 90) (layer Edge.Cuts) (width 0.15))
 (gr_line (start 100 71) (end 100 126.5) (angle 90) (layer Edge.Cuts) (width 0.15))
 (segment (start 149 77.2) (end 148.8 77) (width 0.1524) (layer F.Cu) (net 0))
 (segment (start 124.49 117.84) (end 125.4 117.84) (width 0.1524) (layer B.Cu) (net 1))
 (segment (start 125.4 117.84) (end 126.56 117.84) (width 0.1524) (layer F.Cu) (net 1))
 (segment (start 130.48 125.46) (end 130.48 125.18) (width 0.1524) (layer F.Cu) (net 20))
 (segment (start 127.94 125.46) (end 128.29 125.46) (width 0.1524) (layer B.Cu) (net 34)))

